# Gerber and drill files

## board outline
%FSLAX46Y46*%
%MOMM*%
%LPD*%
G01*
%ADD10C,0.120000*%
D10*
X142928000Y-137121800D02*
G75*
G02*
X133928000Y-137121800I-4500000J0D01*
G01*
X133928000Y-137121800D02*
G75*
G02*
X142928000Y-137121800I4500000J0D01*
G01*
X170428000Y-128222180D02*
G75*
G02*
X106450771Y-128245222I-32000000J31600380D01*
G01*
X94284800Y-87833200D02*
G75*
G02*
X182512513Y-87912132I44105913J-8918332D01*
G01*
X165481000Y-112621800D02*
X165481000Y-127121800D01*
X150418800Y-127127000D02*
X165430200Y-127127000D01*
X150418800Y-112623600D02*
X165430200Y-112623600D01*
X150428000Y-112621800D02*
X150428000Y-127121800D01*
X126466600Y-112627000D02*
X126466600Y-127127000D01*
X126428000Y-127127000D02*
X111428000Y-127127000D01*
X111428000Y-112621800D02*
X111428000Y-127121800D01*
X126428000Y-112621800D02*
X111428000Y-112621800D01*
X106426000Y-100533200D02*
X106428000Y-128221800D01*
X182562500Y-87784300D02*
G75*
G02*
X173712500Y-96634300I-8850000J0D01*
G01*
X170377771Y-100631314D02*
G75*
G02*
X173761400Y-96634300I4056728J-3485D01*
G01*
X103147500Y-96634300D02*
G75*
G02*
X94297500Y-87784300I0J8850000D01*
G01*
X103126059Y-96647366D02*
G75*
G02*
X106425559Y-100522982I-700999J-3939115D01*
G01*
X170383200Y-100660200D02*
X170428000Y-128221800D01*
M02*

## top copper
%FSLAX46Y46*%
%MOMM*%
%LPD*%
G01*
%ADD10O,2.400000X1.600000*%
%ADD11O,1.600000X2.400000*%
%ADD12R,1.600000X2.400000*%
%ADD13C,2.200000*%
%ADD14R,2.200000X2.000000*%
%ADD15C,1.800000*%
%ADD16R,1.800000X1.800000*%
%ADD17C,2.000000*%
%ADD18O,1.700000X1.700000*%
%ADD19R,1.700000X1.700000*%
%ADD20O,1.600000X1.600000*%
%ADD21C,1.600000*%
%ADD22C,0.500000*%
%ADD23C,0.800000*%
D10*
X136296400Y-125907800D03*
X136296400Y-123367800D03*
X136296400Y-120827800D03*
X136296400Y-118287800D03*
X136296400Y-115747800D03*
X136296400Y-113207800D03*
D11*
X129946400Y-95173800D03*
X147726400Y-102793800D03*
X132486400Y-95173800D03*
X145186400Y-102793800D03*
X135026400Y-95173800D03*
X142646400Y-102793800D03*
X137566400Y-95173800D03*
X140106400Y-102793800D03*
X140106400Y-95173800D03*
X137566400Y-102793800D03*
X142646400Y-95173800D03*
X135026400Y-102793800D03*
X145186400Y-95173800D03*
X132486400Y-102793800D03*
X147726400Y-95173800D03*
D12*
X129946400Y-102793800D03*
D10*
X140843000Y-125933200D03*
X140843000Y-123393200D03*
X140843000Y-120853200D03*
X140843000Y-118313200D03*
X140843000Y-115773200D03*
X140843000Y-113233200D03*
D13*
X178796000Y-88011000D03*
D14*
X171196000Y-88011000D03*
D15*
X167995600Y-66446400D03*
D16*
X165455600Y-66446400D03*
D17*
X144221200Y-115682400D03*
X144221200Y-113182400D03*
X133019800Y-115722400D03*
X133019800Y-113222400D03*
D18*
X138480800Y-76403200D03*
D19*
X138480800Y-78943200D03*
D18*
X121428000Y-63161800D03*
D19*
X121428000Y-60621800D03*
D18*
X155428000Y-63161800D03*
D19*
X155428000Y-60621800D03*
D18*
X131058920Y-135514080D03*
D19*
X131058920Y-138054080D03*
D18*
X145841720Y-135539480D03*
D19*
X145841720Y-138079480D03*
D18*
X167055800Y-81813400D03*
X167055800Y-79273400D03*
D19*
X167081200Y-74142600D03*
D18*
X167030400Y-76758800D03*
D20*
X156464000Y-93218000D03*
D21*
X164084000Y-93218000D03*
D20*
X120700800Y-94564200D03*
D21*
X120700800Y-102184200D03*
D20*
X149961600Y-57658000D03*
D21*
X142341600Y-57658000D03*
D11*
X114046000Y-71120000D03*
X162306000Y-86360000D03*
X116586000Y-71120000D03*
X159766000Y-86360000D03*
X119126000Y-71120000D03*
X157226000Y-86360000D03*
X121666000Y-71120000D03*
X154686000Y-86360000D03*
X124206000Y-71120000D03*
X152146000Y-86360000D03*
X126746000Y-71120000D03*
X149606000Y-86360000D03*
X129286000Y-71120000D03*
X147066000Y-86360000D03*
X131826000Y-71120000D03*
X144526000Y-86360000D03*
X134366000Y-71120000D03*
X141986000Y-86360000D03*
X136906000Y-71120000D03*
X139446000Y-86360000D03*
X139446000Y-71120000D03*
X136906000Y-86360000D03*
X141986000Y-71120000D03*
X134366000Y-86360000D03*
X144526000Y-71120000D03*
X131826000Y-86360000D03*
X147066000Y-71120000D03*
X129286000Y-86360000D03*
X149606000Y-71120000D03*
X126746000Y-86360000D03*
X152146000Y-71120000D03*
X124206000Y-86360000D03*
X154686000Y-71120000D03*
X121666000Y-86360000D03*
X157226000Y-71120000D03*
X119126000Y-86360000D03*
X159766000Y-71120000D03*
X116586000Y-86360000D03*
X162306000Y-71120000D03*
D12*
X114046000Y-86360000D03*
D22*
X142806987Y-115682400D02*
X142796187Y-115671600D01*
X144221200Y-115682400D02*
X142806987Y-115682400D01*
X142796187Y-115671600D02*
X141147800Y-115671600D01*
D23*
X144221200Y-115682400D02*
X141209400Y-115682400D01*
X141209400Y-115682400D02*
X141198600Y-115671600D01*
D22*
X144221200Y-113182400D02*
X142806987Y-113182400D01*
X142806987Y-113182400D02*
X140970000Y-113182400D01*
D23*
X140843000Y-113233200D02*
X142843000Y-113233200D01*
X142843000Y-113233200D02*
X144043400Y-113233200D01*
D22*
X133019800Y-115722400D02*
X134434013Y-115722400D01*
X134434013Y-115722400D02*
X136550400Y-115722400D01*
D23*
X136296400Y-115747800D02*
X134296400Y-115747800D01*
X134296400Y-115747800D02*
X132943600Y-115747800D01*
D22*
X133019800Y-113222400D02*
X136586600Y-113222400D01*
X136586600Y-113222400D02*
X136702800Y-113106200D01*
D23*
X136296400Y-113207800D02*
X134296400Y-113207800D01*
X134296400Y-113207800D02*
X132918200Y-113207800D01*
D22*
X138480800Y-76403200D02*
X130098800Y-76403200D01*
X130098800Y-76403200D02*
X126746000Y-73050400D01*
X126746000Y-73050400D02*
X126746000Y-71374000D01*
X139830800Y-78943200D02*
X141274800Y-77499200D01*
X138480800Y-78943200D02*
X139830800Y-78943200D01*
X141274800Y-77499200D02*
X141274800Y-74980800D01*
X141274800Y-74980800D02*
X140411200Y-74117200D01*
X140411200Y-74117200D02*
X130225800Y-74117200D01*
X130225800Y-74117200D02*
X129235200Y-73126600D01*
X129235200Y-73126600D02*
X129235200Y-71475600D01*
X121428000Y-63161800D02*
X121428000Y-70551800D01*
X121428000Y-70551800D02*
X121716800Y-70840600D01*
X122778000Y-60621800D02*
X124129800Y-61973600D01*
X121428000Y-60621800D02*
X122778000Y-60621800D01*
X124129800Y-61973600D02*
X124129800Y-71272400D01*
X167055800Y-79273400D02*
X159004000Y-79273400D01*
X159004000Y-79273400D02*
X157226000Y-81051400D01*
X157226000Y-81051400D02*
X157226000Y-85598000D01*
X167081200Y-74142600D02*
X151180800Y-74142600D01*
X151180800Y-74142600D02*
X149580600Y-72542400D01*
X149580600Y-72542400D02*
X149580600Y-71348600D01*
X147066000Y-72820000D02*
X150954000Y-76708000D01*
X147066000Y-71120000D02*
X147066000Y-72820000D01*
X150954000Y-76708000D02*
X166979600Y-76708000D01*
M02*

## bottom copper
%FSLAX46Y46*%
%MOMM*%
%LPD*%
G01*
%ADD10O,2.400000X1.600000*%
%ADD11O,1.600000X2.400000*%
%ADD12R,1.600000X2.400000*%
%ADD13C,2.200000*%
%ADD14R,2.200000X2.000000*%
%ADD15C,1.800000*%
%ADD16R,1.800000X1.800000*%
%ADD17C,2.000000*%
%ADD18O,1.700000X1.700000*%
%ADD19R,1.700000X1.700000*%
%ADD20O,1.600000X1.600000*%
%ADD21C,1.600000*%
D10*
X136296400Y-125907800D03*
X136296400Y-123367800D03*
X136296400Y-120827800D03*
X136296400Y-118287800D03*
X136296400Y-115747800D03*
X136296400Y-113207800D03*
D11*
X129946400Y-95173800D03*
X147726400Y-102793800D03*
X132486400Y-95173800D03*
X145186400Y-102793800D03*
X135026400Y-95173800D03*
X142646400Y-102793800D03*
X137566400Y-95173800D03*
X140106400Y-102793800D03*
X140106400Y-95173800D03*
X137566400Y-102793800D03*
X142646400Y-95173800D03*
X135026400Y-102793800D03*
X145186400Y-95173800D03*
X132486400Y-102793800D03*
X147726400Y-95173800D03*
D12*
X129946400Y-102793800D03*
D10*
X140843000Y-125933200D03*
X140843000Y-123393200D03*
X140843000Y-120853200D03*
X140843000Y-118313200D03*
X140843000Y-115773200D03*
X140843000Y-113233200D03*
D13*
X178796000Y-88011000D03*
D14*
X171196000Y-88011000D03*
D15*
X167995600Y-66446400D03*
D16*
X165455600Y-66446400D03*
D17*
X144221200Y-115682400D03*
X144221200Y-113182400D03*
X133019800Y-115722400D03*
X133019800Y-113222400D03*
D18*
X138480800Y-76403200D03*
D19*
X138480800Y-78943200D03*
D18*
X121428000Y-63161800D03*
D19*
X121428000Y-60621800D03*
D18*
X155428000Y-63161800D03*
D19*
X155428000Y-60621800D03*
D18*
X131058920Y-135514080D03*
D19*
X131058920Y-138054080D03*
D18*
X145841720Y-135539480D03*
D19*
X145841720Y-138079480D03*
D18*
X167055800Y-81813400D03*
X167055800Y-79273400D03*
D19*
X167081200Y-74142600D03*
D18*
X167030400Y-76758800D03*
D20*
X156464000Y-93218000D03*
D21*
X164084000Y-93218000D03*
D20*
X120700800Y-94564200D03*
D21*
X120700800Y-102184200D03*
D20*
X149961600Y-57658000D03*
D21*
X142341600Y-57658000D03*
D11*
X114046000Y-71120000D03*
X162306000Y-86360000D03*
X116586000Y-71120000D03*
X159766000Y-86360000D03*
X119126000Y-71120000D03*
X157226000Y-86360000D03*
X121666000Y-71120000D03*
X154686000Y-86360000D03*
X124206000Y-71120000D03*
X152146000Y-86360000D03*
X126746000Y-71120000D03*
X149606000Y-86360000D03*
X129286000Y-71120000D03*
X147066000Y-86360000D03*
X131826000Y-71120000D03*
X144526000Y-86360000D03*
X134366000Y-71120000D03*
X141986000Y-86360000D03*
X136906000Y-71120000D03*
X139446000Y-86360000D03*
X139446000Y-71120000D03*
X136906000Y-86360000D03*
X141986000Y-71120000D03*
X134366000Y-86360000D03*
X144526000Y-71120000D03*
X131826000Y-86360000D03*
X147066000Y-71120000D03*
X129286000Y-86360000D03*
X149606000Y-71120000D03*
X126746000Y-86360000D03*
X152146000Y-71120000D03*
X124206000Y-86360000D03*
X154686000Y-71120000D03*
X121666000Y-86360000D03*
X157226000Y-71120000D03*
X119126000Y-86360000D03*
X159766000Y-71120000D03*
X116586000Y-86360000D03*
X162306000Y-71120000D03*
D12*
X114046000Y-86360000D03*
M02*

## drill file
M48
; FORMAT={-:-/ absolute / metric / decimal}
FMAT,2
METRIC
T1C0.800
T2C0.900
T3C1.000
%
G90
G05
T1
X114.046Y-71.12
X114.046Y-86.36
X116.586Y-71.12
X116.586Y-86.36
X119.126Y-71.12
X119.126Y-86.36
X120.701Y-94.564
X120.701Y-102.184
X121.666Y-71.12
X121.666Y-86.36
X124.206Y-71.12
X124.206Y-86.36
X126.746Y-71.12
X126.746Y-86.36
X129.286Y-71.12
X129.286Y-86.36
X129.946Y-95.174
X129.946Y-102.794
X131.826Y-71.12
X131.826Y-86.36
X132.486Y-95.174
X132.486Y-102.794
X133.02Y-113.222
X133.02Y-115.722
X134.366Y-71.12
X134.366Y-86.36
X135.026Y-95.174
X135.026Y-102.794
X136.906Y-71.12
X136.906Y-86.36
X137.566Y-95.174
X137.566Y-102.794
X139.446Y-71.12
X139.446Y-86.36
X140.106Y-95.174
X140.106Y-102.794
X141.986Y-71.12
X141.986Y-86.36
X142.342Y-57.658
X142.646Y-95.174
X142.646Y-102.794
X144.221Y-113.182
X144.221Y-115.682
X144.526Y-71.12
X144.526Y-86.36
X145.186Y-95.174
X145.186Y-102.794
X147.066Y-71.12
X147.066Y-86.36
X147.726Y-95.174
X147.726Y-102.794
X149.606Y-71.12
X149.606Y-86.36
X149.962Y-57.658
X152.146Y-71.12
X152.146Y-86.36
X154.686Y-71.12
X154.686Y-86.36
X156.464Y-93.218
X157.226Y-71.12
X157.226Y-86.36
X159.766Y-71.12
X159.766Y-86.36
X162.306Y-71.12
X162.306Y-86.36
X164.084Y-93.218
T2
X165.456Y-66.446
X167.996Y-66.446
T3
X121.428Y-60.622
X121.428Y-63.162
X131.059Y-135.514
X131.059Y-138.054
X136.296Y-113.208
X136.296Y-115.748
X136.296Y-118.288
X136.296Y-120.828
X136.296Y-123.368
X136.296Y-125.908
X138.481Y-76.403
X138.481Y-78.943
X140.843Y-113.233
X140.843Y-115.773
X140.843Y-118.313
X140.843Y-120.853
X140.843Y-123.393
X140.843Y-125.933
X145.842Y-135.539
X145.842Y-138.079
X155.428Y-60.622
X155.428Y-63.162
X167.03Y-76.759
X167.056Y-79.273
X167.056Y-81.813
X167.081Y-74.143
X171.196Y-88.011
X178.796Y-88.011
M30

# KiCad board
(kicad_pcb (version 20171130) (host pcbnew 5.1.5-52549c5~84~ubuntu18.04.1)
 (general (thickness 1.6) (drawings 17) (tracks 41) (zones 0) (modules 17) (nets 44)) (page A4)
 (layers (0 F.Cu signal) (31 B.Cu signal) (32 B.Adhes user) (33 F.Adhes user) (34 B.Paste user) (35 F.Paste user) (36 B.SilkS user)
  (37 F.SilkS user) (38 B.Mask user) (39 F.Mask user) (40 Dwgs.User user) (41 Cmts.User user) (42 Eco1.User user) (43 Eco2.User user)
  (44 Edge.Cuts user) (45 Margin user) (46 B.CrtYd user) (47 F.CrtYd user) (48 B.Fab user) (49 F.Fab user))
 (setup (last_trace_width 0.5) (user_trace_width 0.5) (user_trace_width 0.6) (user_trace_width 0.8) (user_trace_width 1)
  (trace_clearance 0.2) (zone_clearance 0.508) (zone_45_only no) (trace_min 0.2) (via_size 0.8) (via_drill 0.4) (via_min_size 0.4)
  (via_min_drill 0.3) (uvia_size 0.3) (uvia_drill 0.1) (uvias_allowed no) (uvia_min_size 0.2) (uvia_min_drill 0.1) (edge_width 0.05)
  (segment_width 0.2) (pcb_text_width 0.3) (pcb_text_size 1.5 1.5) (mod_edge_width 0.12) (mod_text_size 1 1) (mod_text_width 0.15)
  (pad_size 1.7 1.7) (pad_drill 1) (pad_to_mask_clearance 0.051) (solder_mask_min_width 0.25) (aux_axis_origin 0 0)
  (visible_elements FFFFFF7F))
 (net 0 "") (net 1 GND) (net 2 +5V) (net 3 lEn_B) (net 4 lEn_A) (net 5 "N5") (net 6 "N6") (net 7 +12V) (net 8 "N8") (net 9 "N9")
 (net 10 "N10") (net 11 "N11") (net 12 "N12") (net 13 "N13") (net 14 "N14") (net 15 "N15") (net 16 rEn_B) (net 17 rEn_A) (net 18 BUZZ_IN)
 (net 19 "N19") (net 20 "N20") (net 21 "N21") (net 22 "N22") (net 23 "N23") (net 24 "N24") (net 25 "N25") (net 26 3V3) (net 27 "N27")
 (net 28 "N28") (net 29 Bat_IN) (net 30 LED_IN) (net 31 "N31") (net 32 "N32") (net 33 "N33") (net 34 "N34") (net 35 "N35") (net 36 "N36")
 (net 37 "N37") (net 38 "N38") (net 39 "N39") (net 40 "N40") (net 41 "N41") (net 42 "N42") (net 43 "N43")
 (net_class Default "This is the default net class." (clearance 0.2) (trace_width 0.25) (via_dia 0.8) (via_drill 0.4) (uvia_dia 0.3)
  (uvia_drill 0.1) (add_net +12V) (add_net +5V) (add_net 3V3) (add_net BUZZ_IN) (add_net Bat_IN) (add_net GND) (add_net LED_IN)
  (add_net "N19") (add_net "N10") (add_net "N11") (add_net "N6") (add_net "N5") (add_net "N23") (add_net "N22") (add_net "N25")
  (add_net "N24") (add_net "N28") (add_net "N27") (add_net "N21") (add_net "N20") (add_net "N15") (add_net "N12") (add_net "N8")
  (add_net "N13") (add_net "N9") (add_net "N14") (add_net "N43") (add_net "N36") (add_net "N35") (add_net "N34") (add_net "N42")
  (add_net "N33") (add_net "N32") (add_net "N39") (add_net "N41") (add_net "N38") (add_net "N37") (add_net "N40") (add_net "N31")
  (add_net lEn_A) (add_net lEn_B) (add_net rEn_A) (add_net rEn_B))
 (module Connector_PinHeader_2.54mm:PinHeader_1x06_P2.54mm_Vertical (layer F.Cu) (at 136.2964 113.2078)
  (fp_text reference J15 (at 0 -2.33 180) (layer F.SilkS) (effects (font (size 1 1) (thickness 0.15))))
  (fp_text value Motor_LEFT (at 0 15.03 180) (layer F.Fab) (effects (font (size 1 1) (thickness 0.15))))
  (pad 6 thru_hole oval (at 0 12.7) (size 2.4 1.6) (drill 1) (layers *.Cu *.Mask) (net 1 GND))
  (pad 5 thru_hole oval (at 0 10.16) (size 2.4 1.6) (drill 1) (layers *.Cu *.Mask) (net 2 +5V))
  (pad 4 thru_hole oval (at 0 7.62) (size 2.4 1.6) (drill 1) (layers *.Cu *.Mask) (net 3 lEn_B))
  (pad 3 thru_hole oval (at 0 5.08) (size 2.4 1.6) (drill 1) (layers *.Cu *.Mask) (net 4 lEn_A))
  (pad 2 thru_hole oval (at 0 2.54) (size 2.4 1.6) (drill 1) (layers *.Cu *.Mask) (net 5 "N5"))
  (pad 1 thru_hole oval (at 0 0) (size 2.4 1.6) (drill 1) (layers *.Cu *.Mask) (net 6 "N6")))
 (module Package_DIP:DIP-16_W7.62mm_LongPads (layer F.Cu) (at 129.9464 102.7938 90)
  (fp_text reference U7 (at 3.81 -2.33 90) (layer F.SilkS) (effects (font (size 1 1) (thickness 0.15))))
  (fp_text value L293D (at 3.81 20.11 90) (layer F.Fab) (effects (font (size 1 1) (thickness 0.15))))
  (pad 16 thru_hole oval (at 7.62 0 90) (size 2.4 1.6) (drill 0.8) (layers *.Cu *.Mask) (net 2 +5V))
  (pad 8 thru_hole oval (at 0 17.78 90) (size 2.4 1.6) (drill 0.8) (layers *.Cu *.Mask) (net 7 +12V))
  (pad 15 thru_hole oval (at 7.62 2.54 90) (size 2.4 1.6) (drill 0.8) (layers *.Cu *.Mask) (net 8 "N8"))
  (pad 7 thru_hole oval (at 0 15.24 90) (size 2.4 1.6) (drill 0.8) (layers *.Cu *.Mask) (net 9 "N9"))
  (pad 14 thru_hole oval (at 7.62 5.08 90) (size 2.4 1.6) (drill 0.8) (layers *.Cu *.Mask) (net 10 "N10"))
  (pad 6 thru_hole oval (at 0 12.7 90) (size 2.4 1.6) (drill 0.8) (layers *.Cu *.Mask) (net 6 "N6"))
  (pad 13 thru_hole oval (at 7.62 7.62 90) (size 2.4 1.6) (drill 0.8) (layers *.Cu *.Mask) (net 1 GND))
  (pad 5 thru_hole oval (at 0 10.16 90) (size 2.4 1.6) (drill 0.8) (layers *.Cu *.Mask) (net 1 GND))
  (pad 12 thru_hole oval (at 7.62 10.16 90) (size 2.4 1.6) (drill 0.8) (layers *.Cu *.Mask) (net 1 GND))
  (pad 4 thru_hole oval (at 0 7.62 90) (size 2.4 1.6) (drill 0.8) (layers *.Cu *.Mask) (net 1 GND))
  (pad 11 thru_hole oval (at 7.62 12.7 90) (size 2.4 1.6) (drill 0.8) (layers *.Cu *.Mask) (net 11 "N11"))
  (pad 3 thru_hole oval (at 0 5.08 90) (size 2.4 1.6) (drill 0.8) (layers *.Cu *.Mask) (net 5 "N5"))
  (pad 10 thru_hole oval (at 7.62 15.24 90) (size 2.4 1.6) (drill 0.8) (layers *.Cu *.Mask) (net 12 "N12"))
  (pad 2 thru_hole oval (at 0 2.54 90) (size 2.4 1.6) (drill 0.8) (layers *.Cu *.Mask) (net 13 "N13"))
  (pad 9 thru_hole oval (at 7.62 17.78 90) (size 2.4 1.6) (drill 0.8) (layers *.Cu *.Mask) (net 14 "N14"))
  (pad 1 thru_hole rect (at 0 0 90) (size 2.4 1.6) (drill 0.8) (layers *.Cu *.Mask) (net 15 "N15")))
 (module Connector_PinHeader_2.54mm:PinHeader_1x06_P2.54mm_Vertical (layer F.Cu) (at 140.843 113.2332)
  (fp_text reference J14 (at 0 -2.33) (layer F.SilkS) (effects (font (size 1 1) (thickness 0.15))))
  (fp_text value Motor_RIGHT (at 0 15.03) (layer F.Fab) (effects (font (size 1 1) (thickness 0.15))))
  (pad 6 thru_hole oval (at 0 12.7) (size 2.4 1.6) (drill 1) (layers *.Cu *.Mask) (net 1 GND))
  (pad 5 thru_hole oval (at 0 10.16) (size 2.4 1.6) (drill 1) (layers *.Cu *.Mask) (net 2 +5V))
  (pad 4 thru_hole oval (at 0 7.62) (size 2.4 1.6) (drill 1) (layers *.Cu *.Mask) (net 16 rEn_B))
  (pad 3 thru_hole oval (at 0 5.08) (size 2.4 1.6) (drill 1) (layers *.Cu *.Mask) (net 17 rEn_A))
  (pad 2 thru_hole oval (at 0 2.54) (size 2.4 1.6) (drill 1) (layers *.Cu *.Mask) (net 11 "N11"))
  (pad 1 thru_hole oval (at 0 0) (size 2.4 1.6) (drill 1) (layers *.Cu *.Mask) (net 10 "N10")))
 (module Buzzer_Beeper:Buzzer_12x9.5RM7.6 (layer F.Cu) (at 171.196 88.011)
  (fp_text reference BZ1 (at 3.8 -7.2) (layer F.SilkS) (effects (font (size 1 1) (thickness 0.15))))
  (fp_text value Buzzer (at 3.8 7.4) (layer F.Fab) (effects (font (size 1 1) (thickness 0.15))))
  (pad 2 thru_hole circle (at 7.6 0) (size 2.2 2.2) (drill 1) (layers *.Cu *.Mask) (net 1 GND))
  (pad 1 thru_hole rect (at 0 0) (size 2.2 2) (drill 1) (layers *.Cu *.Mask) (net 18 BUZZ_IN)))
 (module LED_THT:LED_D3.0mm (layer F.Cu) (at 165.4556 66.4464)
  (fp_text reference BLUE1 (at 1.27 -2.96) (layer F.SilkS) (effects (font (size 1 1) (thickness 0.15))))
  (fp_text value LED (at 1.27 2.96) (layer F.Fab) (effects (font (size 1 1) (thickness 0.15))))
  (pad 2 thru_hole circle (at 2.54 0) (size 1.8 1.8) (drill 0.9) (layers *.Cu *.Mask) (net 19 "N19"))
  (pad 1 thru_hole rect (at 0 0) (size 1.8 1.8) (drill 0.9) (layers *.Cu *.Mask) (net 1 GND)))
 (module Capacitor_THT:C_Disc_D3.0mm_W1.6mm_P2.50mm (layer F.Cu) (at 144.2212 113.1824 270)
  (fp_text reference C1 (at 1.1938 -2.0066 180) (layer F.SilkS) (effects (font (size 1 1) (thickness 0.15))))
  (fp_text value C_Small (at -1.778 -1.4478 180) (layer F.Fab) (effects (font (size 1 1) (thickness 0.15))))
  (pad 2 thru_hole circle (at 2.5 0 270) (size 2 2) (drill 0.8) (layers *.Cu *.Mask) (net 11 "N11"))
  (pad 1 thru_hole circle (at 0 0 270) (size 2 2) (drill 0.8) (layers *.Cu *.Mask) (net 10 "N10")))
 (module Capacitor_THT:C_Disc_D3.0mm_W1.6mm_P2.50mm (layer F.Cu) (at 133.0198 113.2224 270)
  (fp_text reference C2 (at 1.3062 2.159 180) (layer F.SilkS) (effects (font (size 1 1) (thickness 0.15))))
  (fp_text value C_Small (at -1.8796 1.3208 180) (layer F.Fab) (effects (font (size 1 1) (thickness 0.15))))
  (pad 2 thru_hole circle (at 2.5 0 270) (size 2 2) (drill 0.8) (layers *.Cu *.Mask) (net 5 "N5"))
  (pad 1 thru_hole circle (at 0 0 270) (size 2 2) (drill 0.8) (layers *.Cu *.Mask) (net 6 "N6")))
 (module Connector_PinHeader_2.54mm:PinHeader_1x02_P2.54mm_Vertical (layer F.Cu) (at 138.4808 78.9432 180)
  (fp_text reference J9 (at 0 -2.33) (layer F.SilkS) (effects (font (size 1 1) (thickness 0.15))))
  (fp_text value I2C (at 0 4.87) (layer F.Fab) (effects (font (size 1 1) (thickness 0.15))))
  (pad 2 thru_hole oval (at 0 2.54 180) (size 1.7 1.7) (drill 1) (layers *.Cu *.Mask) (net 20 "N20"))
  (pad 1 thru_hole rect (at 0 0 180) (size 1.7 1.7) (drill 1) (layers *.Cu *.Mask) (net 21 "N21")))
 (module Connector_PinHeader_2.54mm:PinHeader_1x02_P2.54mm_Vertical (layer F.Cu) (at 121.428 60.6218)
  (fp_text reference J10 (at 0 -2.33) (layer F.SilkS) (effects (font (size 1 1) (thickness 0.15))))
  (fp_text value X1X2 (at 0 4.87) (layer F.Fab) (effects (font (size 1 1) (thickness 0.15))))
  (pad 2 thru_hole oval (at 0 2.54) (size 1.7 1.7) (drill 1) (layers *.Cu *.Mask) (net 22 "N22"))
  (pad 1 thru_hole rect (at 0 0) (size 1.7 1.7) (drill 1) (layers *.Cu *.Mask) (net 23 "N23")))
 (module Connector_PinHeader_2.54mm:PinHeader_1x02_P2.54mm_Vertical (layer F.Cu) (at 155.428 60.6218)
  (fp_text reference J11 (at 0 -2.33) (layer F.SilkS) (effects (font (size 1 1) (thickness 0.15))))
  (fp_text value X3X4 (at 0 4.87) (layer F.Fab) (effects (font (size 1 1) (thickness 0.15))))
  (pad 2 thru_hole oval (at 0 2.54) (size 1.7 1.7) (drill 1) (layers *.Cu *.Mask) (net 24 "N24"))
  (pad 1 thru_hole rect (at 0 0) (size 1.7 1.7) (drill 1) (layers *.Cu *.Mask) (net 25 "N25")))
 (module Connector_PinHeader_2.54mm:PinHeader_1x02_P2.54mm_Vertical (layer F.Cu) (at 131.05892 138.05408 180)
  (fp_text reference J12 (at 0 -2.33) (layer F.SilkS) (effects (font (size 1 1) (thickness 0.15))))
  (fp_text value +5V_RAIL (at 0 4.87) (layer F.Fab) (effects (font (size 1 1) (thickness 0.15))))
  (pad 2 thru_hole oval (at 0 2.54 180) (size 1.7 1.7) (drill 1) (layers *.Cu *.Mask) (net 1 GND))
  (pad 1 thru_hole rect (at 0 0 180) (size 1.7 1.7) (drill 1) (layers *.Cu *.Mask) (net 2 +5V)))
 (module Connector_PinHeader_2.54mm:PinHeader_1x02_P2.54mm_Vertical (layer F.Cu) (at 145.84172 138.07948 180)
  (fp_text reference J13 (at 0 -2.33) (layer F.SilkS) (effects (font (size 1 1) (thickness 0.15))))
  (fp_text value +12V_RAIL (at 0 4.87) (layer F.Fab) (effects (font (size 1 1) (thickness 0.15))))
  (pad 2 thru_hole oval (at 0 2.54 180) (size 1.7 1.7) (drill 1) (layers *.Cu *.Mask) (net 1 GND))
  (pad 1 thru_hole rect (at 0 0 180) (size 1.7 1.7) (drill 1) (layers *.Cu *.Mask) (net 7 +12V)))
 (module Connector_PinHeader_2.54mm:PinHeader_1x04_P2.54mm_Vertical (layer F.Cu) (at 167.0558 74.1934)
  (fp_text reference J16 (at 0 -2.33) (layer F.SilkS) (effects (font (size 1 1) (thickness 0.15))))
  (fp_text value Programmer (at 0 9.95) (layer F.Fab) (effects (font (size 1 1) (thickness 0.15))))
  (pad 4 thru_hole oval (at 0 7.62) (size 1.7 1.7) (drill 1) (layers *.Cu *.Mask) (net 1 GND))
  (pad 3 thru_hole oval (at 0 5.08) (size 1.7 1.7) (drill 1) (layers *.Cu *.Mask) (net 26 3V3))
  (pad 2 thru_hole rect (at 0.0254 -0.0508) (size 1.7 1.7) (drill 1) (layers *.Cu *.Mask) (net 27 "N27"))
  (pad 1 thru_hole oval (at -0.0254 2.5654) (size 1.7 1.7) (drill 1) (layers *.Cu *.Mask) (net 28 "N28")))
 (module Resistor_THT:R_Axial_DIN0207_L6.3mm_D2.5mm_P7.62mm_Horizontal (layer F.Cu) (at 164.084 93.218 180)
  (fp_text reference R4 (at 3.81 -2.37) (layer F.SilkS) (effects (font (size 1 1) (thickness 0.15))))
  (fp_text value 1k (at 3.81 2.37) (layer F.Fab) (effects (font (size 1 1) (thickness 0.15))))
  (pad 2 thru_hole oval (at 7.62 0 180) (size 1.6 1.6) (drill 0.8) (layers *.Cu *.Mask) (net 1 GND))
  (pad 1 thru_hole circle (at 0 0 180) (size 1.6 1.6) (drill 0.8) (layers *.Cu *.Mask) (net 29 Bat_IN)))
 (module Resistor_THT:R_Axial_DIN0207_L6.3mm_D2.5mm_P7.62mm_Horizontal (layer F.Cu) (at 120.7008 102.1842 90)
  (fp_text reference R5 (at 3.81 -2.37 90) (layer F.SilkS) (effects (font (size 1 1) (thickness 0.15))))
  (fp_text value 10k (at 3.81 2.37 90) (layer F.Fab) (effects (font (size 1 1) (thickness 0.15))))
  (pad 2 thru_hole oval (at 7.62 0 90) (size 1.6 1.6) (drill 0.8) (layers *.Cu *.Mask) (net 29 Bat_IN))
  (pad 1 thru_hole circle (at 0 0 90) (size 1.6 1.6) (drill 0.8) (layers *.Cu *.Mask) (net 7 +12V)))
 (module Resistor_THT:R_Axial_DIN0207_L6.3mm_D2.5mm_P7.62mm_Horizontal (layer F.Cu) (at 142.3416 57.658)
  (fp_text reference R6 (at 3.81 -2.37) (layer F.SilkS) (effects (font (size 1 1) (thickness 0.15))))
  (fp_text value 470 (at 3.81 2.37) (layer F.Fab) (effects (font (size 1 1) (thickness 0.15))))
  (pad 2 thru_hole oval (at 7.62 0) (size 1.6 1.6) (drill 0.8) (layers *.Cu *.Mask) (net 19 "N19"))
  (pad 1 thru_hole circle (at 0 0) (size 1.6 1.6) (drill 0.8) (layers *.Cu *.Mask) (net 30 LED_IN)))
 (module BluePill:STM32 (layer F.Cu) (at 114.046 86.36 90)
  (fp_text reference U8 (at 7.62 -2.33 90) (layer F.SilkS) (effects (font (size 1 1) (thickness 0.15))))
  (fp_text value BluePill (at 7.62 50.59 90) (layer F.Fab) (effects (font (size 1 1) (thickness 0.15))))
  (pad 3V3 thru_hole oval (at 15.24 0 90) (size 2.4 1.6) (drill 0.8) (layers *.Cu *.Mask) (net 26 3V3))
  (pad GND thru_hole oval (at 0 48.26 90) (size 2.4 1.6) (drill 0.8) (layers *.Cu *.Mask) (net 1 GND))
  (pad GND thru_hole oval (at 15.24 2.54 90) (size 2.4 1.6) (drill 0.8) (layers *.Cu *.Mask) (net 1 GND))
  (pad GND thru_hole oval (at 0 45.72 90) (size 2.4 1.6) (drill 0.8) (layers *.Cu *.Mask) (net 1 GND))
  (pad 5V thru_hole oval (at 15.24 5.08 90) (size 2.4 1.6) (drill 0.8) (layers *.Cu *.Mask) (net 2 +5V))
  (pad 3V3 thru_hole oval (at 0 43.18 90) (size 2.4 1.6) (drill 0.8) (layers *.Cu *.Mask) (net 26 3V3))
  (pad 46 thru_hole oval (at 15.24 7.62 90) (size 2.4 1.6) (drill 0.8) (layers *.Cu *.Mask) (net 22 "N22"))
  (pad 7 thru_hole oval (at 0 40.64 90) (size 2.4 1.6) (drill 0.8) (layers *.Cu *.Mask) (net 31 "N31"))
  (pad 45 thru_hole oval (at 15.24 10.16 90) (size 2.4 1.6) (drill 0.8) (layers *.Cu *.Mask) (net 23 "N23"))
  (pad 22 thru_hole oval (at 0 38.1 90) (size 2.4 1.6) (drill 0.8) (layers *.Cu *.Mask) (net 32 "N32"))
  (pad 43 thru_hole oval (at 15.24 12.7 90) (size 2.4 1.6) (drill 0.8) (layers *.Cu *.Mask) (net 20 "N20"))
  (pad 21 thru_hole oval (at 0 35.56 90) (size 2.4 1.6) (drill 0.8) (layers *.Cu *.Mask) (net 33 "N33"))
  (pad 42 thru_hole oval (at 15.24 15.24 90) (size 2.4 1.6) (drill 0.8) (layers *.Cu *.Mask) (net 21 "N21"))
  (pad 19 thru_hole oval (at 0 33.02 90) (size 2.4 1.6) (drill 0.8) (layers *.Cu *.Mask) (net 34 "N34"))
  (pad 41 thru_hole oval (at 15.24 17.78 90) (size 2.4 1.6) (drill 0.8) (layers *.Cu *.Mask) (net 24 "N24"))
  (pad 18 thru_hole oval (at 0 30.48 90) (size 2.4 1.6) (drill 0.8) (layers *.Cu *.Mask) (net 29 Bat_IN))
  (pad 40 thru_hole oval (at 15.24 20.32 90) (size 2.4 1.6) (drill 0.8) (layers *.Cu *.Mask) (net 25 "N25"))
  (pad 17 thru_hole oval (at 0 27.94 90) (size 2.4 1.6) (drill 0.8) (layers *.Cu *.Mask) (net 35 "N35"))
  (pad 39 thru_hole oval (at 15.24 22.86 90) (size 2.4 1.6) (drill 0.8) (layers *.Cu *.Mask) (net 30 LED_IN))
  (pad 16 thru_hole oval (at 0 25.4 90) (size 2.4 1.6) (drill 0.8) (layers *.Cu *.Mask) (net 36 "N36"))
  (pad 38 thru_hole oval (at 15.24 25.4 90) (size 2.4 1.6) (drill 0.8) (layers *.Cu *.Mask) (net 18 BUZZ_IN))
  (pad 15 thru_hole oval (at 0 22.86 90) (size 2.4 1.6) (drill 0.8) (layers *.Cu *.Mask) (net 13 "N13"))
  (pad 33 thru_hole oval (at 15.24 27.94 90) (size 2.4 1.6) (drill 0.8) (layers *.Cu *.Mask) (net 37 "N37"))
  (pad 14 thru_hole oval (at 0 20.32 90) (size 2.4 1.6) (drill 0.8) (layers *.Cu *.Mask) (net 9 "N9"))
  (pad 32 thru_hole oval (at 15.24 30.48 90) (size 2.4 1.6) (drill 0.8) (layers *.Cu *.Mask) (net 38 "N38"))
  (pad 13 thru_hole oval (at 0 17.78 90) (size 2.4 1.6) (drill 0.8) (layers *.Cu *.Mask) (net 15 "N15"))
  (pad 31 thru_hole oval (at 15.24 33.02 90) (size 2.4 1.6) (drill 0.8) (layers *.Cu *.Mask) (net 28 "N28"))
  (pad 12 thru_hole oval (at 0 15.24 90) (size 2.4 1.6) (drill 0.8) (layers *.Cu *.Mask) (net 12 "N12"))
  (pad 30 thru_hole oval (at 15.24 35.56 90) (size 2.4 1.6) (drill 0.8) (layers *.Cu *.Mask) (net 27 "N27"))
  (pad 11 thru_hole oval (at 0 12.7 90) (size 2.4 1.6) (drill 0.8) (layers *.Cu *.Mask) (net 8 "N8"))
  (pad 29 thru_hole oval (at 15.24 38.1 90) (size 2.4 1.6) (drill 0.8) (layers *.Cu *.Mask) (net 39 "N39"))
  (pad 10 thru_hole oval (at 0 10.16 90) (size 2.4 1.6) (drill 0.8) (layers *.Cu *.Mask) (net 14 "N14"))
  (pad 28 thru_hole oval (at 15.24 40.64 90) (size 2.4 1.6) (drill 0.8) (layers *.Cu *.Mask) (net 4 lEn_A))
  (pad 4 thru_hole oval (at 0 7.62 90) (size 2.4 1.6) (drill 0.8) (layers *.Cu *.Mask) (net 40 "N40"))
  (pad 27 thru_hole oval (at 15.24 43.18 90) (size 2.4 1.6) (drill 0.8) (layers *.Cu *.Mask) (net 3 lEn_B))
  (pad 3 thru_hole oval (at 0 5.08 90) (size 2.4 1.6) (drill 0.8) (layers *.Cu *.Mask) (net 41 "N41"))
  (pad 26 thru_hole oval (at 15.24 45.72 90) (size 2.4 1.6) (drill 0.8) (layers *.Cu *.Mask) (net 17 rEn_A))
  (pad 2 thru_hole oval (at 0 2.54 90) (size 2.4 1.6) (drill 0.8) (layers *.Cu *.Mask) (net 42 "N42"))
  (pad 25 thru_hole oval (at 15.24 48.26 90) (size 2.4 1.6) (drill 0.8) (layers *.Cu *.Mask) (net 16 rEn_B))
  (pad 1 thru_hole rect (at 0 0 90) (size 2.4 1.6) (drill 0.8) (layers *.Cu *.Mask) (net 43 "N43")))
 (gr_circle (center 138.428 137.1218) (end 142.928 137.1218) (layer Edge.Cuts) (width 0.12))
 (gr_arc (start 138.428 96.6218) (end 170.428 128.22218) (angle 90.67873161) (layer Edge.Cuts) (width 0.12))
 (gr_arc (start 138.390713 96.751532) (end 182.512513 87.912132) (angle -157.2400599) (layer Edge.Cuts) (width 0.12))
 (gr_line (start 165.481 112.6218) (end 165.481 127.1218) (layer Edge.Cuts) (width 0.12))
 (gr_line (start 150.4188 127.127) (end 165.4302 127.127) (layer Edge.Cuts) (width 0.12))
 (gr_line (start 150.4188 112.6236) (end 165.4302 112.6236) (layer Edge.Cuts) (width 0.12))
 (gr_line (start 150.428 112.6218) (end 150.428 127.1218) (layer Edge.Cuts) (width 0.12))
 (gr_line (start 126.4666 112.627) (end 126.4666 127.127) (layer Edge.Cuts) (width 0.12))
 (gr_line (start 126.428 127.127) (end 111.428 127.127) (layer Edge.Cuts) (width 0.12))
 (gr_line (start 111.428 112.6218) (end 111.428 127.1218) (layer Edge.Cuts) (width 0.12))
 (gr_line (start 126.428 112.6218) (end 111.428 112.6218) (layer Edge.Cuts) (width 0.12))
 (gr_line (start 106.426 100.5332) (end 106.428 128.2218) (layer Edge.Cuts) (width 0.12))
 (gr_arc (start 173.7125 87.7843) (end 173.7125 96.6343) (angle -90) (layer Edge.Cuts) (width 0.12))
 (gr_arc (start 174.434499 100.634799) (end 173.7614 96.6343) (angle -80.4) (layer Edge.Cuts) (width 0.12))
 (gr_arc (start 103.1475 87.7843) (end 94.2975 87.7843) (angle -90) (layer Edge.Cuts) (width 0.12))
 (gr_arc (start 102.42506 100.586481) (end 106.425559 100.522982) (angle -79) (layer Edge.Cuts) (width 0.12))
 (gr_line (start 170.3832 100.6602) (end 170.428 128.2218) (layer Edge.Cuts) (width 0.12))
 (segment (start 142.806987 115.6824) (end 142.796187 115.6716) (width 0.5) (layer F.Cu) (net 11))
 (segment (start 144.2212 115.6824) (end 142.806987 115.6824) (width 0.5) (layer F.Cu) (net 11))
 (segment (start 142.796187 115.6716) (end 141.1478 115.6716) (width 0.5) (layer F.Cu) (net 11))
 (segment (start 144.2212 115.6824) (end 141.2094 115.6824) (width 0.8) (layer F.Cu) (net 11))
 (segment (start 141.2094 115.6824) (end 141.1986 115.6716) (width 0.8) (layer F.Cu) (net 11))
 (segment (start 144.2212 113.1824) (end 142.806987 113.1824) (width 0.5) (layer F.Cu) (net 10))
 (segment (start 142.806987 113.1824) (end 140.97 113.1824) (width 0.5) (layer F.Cu) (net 10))
 (segment (start 140.843 113.2332) (end 142.843 113.2332) (width 0.8) (layer F.Cu) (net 10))
 (segment (start 142.843 113.2332) (end 144.0434 113.2332) (width 0.8) (layer F.Cu) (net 10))
 (segment (start 133.0198 115.7224) (end 134.434013 115.7224) (width 0.5) (layer F.Cu) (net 5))
 (segment (start 134.434013 115.7224) (end 136.5504 115.7224) (width 0.5) (layer F.Cu) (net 5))
 (segment (start 136.2964 115.7478) (end 134.2964 115.7478) (width 0.8) (layer F.Cu) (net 5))
 (segment (start 134.2964 115.7478) (end 132.9436 115.7478) (width 0.8) (layer F.Cu) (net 5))
 (segment (start 133.0198 113.2224) (end 136.5866 113.2224) (width 0.5) (layer F.Cu) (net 6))
 (segment (start 136.5866 113.2224) (end 136.7028 113.1062) (width 0.5) (layer F.Cu) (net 6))
 (segment (start 136.2964 113.2078) (end 134.2964 113.2078) (width 0.8) (layer F.Cu) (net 6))
 (segment (start 134.2964 113.2078) (end 132.9182 113.2078) (width 0.8) (layer F.Cu) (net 6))
 (segment (start 138.4808 76.4032) (end 130.0988 76.4032) (width 0.5) (layer F.Cu) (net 20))
 (segment (start 130.0988 76.4032) (end 126.746 73.0504) (width 0.5) (layer F.Cu) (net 20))
 (segment (start 126.746 73.0504) (end 126.746 71.374) (width 0.5) (layer F.Cu) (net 20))
 (segment (start 139.8308 78.9432) (end 141.2748 77.4992) (width 0.5) (layer F.Cu) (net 21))
 (segment (start 138.4808 78.9432) (end 139.8308 78.9432) (width 0.5) (layer F.Cu) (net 21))
 (segment (start 141.2748 77.4992) (end 141.2748 74.9808) (width 0.5) (layer F.Cu) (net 21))
 (segment (start 141.2748 74.9808) (end 140.4112 74.1172) (width 0.5) (layer F.Cu) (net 21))
 (segment (start 140.4112 74.1172) (end 130.2258 74.1172) (width 0.5) (layer F.Cu) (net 21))
 (segment (start 130.2258 74.1172) (end 129.2352 73.1266) (width 0.5) (layer F.Cu) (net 21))
 (segment (start 129.2352 73.1266) (end 129.2352 71.4756) (width 0.5) (layer F.Cu) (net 21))
 (segment (start 121.428 63.1618) (end 121.428 70.5518) (width 0.5) (layer F.Cu) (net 22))
 (segment (start 121.428 70.5518) (end 121.7168 70.8406) (width 0.5) (layer F.Cu) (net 22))
 (segment (start 122.778 60.6218) (end 124.1298 61.9736) (width 0.5) (layer F.Cu) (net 23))
 (segment (start 121.428 60.6218) (end 122.778 60.6218) (width 0.5) (layer F.Cu) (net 23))
 (segment (start 124.1298 61.9736) (end 124.1298 71.2724) (width 0.5) (layer F.Cu) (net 23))
 (segment (start 167.0558 79.2734) (end 159.004 79.2734) (width 0.5) (layer F.Cu) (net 26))
 (segment (start 159.004 79.2734) (end 157.226 81.0514) (width 0.5) (layer F.Cu) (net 26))
 (segment (start 157.226 81.0514) (end 157.226 85.598) (width 0.5) (layer F.Cu) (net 26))
 (segment (start 167.0812 74.1426) (end 151.1808 74.1426) (width 0.5) (layer F.Cu) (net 27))
 (segment (start 151.1808 74.1426) (end 149.5806 72.5424) (width 0.5) (layer F.Cu) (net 27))
 (segment (start 149.5806 72.5424) (end 149.5806 71.3486) (width 0.5) (layer F.Cu) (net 27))
 (segment (start 147.066 72.82) (end 150.954 76.708) (width 0.5) (layer F.Cu) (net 28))
 (segment (start 147.066 71.12) (end 147.066 72.82) (width 0.5) (layer F.Cu) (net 28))
 (segment (start 150.954 76.708) (end 166.9796 76.708) (width 0.5) (layer F.Cu) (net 28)))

